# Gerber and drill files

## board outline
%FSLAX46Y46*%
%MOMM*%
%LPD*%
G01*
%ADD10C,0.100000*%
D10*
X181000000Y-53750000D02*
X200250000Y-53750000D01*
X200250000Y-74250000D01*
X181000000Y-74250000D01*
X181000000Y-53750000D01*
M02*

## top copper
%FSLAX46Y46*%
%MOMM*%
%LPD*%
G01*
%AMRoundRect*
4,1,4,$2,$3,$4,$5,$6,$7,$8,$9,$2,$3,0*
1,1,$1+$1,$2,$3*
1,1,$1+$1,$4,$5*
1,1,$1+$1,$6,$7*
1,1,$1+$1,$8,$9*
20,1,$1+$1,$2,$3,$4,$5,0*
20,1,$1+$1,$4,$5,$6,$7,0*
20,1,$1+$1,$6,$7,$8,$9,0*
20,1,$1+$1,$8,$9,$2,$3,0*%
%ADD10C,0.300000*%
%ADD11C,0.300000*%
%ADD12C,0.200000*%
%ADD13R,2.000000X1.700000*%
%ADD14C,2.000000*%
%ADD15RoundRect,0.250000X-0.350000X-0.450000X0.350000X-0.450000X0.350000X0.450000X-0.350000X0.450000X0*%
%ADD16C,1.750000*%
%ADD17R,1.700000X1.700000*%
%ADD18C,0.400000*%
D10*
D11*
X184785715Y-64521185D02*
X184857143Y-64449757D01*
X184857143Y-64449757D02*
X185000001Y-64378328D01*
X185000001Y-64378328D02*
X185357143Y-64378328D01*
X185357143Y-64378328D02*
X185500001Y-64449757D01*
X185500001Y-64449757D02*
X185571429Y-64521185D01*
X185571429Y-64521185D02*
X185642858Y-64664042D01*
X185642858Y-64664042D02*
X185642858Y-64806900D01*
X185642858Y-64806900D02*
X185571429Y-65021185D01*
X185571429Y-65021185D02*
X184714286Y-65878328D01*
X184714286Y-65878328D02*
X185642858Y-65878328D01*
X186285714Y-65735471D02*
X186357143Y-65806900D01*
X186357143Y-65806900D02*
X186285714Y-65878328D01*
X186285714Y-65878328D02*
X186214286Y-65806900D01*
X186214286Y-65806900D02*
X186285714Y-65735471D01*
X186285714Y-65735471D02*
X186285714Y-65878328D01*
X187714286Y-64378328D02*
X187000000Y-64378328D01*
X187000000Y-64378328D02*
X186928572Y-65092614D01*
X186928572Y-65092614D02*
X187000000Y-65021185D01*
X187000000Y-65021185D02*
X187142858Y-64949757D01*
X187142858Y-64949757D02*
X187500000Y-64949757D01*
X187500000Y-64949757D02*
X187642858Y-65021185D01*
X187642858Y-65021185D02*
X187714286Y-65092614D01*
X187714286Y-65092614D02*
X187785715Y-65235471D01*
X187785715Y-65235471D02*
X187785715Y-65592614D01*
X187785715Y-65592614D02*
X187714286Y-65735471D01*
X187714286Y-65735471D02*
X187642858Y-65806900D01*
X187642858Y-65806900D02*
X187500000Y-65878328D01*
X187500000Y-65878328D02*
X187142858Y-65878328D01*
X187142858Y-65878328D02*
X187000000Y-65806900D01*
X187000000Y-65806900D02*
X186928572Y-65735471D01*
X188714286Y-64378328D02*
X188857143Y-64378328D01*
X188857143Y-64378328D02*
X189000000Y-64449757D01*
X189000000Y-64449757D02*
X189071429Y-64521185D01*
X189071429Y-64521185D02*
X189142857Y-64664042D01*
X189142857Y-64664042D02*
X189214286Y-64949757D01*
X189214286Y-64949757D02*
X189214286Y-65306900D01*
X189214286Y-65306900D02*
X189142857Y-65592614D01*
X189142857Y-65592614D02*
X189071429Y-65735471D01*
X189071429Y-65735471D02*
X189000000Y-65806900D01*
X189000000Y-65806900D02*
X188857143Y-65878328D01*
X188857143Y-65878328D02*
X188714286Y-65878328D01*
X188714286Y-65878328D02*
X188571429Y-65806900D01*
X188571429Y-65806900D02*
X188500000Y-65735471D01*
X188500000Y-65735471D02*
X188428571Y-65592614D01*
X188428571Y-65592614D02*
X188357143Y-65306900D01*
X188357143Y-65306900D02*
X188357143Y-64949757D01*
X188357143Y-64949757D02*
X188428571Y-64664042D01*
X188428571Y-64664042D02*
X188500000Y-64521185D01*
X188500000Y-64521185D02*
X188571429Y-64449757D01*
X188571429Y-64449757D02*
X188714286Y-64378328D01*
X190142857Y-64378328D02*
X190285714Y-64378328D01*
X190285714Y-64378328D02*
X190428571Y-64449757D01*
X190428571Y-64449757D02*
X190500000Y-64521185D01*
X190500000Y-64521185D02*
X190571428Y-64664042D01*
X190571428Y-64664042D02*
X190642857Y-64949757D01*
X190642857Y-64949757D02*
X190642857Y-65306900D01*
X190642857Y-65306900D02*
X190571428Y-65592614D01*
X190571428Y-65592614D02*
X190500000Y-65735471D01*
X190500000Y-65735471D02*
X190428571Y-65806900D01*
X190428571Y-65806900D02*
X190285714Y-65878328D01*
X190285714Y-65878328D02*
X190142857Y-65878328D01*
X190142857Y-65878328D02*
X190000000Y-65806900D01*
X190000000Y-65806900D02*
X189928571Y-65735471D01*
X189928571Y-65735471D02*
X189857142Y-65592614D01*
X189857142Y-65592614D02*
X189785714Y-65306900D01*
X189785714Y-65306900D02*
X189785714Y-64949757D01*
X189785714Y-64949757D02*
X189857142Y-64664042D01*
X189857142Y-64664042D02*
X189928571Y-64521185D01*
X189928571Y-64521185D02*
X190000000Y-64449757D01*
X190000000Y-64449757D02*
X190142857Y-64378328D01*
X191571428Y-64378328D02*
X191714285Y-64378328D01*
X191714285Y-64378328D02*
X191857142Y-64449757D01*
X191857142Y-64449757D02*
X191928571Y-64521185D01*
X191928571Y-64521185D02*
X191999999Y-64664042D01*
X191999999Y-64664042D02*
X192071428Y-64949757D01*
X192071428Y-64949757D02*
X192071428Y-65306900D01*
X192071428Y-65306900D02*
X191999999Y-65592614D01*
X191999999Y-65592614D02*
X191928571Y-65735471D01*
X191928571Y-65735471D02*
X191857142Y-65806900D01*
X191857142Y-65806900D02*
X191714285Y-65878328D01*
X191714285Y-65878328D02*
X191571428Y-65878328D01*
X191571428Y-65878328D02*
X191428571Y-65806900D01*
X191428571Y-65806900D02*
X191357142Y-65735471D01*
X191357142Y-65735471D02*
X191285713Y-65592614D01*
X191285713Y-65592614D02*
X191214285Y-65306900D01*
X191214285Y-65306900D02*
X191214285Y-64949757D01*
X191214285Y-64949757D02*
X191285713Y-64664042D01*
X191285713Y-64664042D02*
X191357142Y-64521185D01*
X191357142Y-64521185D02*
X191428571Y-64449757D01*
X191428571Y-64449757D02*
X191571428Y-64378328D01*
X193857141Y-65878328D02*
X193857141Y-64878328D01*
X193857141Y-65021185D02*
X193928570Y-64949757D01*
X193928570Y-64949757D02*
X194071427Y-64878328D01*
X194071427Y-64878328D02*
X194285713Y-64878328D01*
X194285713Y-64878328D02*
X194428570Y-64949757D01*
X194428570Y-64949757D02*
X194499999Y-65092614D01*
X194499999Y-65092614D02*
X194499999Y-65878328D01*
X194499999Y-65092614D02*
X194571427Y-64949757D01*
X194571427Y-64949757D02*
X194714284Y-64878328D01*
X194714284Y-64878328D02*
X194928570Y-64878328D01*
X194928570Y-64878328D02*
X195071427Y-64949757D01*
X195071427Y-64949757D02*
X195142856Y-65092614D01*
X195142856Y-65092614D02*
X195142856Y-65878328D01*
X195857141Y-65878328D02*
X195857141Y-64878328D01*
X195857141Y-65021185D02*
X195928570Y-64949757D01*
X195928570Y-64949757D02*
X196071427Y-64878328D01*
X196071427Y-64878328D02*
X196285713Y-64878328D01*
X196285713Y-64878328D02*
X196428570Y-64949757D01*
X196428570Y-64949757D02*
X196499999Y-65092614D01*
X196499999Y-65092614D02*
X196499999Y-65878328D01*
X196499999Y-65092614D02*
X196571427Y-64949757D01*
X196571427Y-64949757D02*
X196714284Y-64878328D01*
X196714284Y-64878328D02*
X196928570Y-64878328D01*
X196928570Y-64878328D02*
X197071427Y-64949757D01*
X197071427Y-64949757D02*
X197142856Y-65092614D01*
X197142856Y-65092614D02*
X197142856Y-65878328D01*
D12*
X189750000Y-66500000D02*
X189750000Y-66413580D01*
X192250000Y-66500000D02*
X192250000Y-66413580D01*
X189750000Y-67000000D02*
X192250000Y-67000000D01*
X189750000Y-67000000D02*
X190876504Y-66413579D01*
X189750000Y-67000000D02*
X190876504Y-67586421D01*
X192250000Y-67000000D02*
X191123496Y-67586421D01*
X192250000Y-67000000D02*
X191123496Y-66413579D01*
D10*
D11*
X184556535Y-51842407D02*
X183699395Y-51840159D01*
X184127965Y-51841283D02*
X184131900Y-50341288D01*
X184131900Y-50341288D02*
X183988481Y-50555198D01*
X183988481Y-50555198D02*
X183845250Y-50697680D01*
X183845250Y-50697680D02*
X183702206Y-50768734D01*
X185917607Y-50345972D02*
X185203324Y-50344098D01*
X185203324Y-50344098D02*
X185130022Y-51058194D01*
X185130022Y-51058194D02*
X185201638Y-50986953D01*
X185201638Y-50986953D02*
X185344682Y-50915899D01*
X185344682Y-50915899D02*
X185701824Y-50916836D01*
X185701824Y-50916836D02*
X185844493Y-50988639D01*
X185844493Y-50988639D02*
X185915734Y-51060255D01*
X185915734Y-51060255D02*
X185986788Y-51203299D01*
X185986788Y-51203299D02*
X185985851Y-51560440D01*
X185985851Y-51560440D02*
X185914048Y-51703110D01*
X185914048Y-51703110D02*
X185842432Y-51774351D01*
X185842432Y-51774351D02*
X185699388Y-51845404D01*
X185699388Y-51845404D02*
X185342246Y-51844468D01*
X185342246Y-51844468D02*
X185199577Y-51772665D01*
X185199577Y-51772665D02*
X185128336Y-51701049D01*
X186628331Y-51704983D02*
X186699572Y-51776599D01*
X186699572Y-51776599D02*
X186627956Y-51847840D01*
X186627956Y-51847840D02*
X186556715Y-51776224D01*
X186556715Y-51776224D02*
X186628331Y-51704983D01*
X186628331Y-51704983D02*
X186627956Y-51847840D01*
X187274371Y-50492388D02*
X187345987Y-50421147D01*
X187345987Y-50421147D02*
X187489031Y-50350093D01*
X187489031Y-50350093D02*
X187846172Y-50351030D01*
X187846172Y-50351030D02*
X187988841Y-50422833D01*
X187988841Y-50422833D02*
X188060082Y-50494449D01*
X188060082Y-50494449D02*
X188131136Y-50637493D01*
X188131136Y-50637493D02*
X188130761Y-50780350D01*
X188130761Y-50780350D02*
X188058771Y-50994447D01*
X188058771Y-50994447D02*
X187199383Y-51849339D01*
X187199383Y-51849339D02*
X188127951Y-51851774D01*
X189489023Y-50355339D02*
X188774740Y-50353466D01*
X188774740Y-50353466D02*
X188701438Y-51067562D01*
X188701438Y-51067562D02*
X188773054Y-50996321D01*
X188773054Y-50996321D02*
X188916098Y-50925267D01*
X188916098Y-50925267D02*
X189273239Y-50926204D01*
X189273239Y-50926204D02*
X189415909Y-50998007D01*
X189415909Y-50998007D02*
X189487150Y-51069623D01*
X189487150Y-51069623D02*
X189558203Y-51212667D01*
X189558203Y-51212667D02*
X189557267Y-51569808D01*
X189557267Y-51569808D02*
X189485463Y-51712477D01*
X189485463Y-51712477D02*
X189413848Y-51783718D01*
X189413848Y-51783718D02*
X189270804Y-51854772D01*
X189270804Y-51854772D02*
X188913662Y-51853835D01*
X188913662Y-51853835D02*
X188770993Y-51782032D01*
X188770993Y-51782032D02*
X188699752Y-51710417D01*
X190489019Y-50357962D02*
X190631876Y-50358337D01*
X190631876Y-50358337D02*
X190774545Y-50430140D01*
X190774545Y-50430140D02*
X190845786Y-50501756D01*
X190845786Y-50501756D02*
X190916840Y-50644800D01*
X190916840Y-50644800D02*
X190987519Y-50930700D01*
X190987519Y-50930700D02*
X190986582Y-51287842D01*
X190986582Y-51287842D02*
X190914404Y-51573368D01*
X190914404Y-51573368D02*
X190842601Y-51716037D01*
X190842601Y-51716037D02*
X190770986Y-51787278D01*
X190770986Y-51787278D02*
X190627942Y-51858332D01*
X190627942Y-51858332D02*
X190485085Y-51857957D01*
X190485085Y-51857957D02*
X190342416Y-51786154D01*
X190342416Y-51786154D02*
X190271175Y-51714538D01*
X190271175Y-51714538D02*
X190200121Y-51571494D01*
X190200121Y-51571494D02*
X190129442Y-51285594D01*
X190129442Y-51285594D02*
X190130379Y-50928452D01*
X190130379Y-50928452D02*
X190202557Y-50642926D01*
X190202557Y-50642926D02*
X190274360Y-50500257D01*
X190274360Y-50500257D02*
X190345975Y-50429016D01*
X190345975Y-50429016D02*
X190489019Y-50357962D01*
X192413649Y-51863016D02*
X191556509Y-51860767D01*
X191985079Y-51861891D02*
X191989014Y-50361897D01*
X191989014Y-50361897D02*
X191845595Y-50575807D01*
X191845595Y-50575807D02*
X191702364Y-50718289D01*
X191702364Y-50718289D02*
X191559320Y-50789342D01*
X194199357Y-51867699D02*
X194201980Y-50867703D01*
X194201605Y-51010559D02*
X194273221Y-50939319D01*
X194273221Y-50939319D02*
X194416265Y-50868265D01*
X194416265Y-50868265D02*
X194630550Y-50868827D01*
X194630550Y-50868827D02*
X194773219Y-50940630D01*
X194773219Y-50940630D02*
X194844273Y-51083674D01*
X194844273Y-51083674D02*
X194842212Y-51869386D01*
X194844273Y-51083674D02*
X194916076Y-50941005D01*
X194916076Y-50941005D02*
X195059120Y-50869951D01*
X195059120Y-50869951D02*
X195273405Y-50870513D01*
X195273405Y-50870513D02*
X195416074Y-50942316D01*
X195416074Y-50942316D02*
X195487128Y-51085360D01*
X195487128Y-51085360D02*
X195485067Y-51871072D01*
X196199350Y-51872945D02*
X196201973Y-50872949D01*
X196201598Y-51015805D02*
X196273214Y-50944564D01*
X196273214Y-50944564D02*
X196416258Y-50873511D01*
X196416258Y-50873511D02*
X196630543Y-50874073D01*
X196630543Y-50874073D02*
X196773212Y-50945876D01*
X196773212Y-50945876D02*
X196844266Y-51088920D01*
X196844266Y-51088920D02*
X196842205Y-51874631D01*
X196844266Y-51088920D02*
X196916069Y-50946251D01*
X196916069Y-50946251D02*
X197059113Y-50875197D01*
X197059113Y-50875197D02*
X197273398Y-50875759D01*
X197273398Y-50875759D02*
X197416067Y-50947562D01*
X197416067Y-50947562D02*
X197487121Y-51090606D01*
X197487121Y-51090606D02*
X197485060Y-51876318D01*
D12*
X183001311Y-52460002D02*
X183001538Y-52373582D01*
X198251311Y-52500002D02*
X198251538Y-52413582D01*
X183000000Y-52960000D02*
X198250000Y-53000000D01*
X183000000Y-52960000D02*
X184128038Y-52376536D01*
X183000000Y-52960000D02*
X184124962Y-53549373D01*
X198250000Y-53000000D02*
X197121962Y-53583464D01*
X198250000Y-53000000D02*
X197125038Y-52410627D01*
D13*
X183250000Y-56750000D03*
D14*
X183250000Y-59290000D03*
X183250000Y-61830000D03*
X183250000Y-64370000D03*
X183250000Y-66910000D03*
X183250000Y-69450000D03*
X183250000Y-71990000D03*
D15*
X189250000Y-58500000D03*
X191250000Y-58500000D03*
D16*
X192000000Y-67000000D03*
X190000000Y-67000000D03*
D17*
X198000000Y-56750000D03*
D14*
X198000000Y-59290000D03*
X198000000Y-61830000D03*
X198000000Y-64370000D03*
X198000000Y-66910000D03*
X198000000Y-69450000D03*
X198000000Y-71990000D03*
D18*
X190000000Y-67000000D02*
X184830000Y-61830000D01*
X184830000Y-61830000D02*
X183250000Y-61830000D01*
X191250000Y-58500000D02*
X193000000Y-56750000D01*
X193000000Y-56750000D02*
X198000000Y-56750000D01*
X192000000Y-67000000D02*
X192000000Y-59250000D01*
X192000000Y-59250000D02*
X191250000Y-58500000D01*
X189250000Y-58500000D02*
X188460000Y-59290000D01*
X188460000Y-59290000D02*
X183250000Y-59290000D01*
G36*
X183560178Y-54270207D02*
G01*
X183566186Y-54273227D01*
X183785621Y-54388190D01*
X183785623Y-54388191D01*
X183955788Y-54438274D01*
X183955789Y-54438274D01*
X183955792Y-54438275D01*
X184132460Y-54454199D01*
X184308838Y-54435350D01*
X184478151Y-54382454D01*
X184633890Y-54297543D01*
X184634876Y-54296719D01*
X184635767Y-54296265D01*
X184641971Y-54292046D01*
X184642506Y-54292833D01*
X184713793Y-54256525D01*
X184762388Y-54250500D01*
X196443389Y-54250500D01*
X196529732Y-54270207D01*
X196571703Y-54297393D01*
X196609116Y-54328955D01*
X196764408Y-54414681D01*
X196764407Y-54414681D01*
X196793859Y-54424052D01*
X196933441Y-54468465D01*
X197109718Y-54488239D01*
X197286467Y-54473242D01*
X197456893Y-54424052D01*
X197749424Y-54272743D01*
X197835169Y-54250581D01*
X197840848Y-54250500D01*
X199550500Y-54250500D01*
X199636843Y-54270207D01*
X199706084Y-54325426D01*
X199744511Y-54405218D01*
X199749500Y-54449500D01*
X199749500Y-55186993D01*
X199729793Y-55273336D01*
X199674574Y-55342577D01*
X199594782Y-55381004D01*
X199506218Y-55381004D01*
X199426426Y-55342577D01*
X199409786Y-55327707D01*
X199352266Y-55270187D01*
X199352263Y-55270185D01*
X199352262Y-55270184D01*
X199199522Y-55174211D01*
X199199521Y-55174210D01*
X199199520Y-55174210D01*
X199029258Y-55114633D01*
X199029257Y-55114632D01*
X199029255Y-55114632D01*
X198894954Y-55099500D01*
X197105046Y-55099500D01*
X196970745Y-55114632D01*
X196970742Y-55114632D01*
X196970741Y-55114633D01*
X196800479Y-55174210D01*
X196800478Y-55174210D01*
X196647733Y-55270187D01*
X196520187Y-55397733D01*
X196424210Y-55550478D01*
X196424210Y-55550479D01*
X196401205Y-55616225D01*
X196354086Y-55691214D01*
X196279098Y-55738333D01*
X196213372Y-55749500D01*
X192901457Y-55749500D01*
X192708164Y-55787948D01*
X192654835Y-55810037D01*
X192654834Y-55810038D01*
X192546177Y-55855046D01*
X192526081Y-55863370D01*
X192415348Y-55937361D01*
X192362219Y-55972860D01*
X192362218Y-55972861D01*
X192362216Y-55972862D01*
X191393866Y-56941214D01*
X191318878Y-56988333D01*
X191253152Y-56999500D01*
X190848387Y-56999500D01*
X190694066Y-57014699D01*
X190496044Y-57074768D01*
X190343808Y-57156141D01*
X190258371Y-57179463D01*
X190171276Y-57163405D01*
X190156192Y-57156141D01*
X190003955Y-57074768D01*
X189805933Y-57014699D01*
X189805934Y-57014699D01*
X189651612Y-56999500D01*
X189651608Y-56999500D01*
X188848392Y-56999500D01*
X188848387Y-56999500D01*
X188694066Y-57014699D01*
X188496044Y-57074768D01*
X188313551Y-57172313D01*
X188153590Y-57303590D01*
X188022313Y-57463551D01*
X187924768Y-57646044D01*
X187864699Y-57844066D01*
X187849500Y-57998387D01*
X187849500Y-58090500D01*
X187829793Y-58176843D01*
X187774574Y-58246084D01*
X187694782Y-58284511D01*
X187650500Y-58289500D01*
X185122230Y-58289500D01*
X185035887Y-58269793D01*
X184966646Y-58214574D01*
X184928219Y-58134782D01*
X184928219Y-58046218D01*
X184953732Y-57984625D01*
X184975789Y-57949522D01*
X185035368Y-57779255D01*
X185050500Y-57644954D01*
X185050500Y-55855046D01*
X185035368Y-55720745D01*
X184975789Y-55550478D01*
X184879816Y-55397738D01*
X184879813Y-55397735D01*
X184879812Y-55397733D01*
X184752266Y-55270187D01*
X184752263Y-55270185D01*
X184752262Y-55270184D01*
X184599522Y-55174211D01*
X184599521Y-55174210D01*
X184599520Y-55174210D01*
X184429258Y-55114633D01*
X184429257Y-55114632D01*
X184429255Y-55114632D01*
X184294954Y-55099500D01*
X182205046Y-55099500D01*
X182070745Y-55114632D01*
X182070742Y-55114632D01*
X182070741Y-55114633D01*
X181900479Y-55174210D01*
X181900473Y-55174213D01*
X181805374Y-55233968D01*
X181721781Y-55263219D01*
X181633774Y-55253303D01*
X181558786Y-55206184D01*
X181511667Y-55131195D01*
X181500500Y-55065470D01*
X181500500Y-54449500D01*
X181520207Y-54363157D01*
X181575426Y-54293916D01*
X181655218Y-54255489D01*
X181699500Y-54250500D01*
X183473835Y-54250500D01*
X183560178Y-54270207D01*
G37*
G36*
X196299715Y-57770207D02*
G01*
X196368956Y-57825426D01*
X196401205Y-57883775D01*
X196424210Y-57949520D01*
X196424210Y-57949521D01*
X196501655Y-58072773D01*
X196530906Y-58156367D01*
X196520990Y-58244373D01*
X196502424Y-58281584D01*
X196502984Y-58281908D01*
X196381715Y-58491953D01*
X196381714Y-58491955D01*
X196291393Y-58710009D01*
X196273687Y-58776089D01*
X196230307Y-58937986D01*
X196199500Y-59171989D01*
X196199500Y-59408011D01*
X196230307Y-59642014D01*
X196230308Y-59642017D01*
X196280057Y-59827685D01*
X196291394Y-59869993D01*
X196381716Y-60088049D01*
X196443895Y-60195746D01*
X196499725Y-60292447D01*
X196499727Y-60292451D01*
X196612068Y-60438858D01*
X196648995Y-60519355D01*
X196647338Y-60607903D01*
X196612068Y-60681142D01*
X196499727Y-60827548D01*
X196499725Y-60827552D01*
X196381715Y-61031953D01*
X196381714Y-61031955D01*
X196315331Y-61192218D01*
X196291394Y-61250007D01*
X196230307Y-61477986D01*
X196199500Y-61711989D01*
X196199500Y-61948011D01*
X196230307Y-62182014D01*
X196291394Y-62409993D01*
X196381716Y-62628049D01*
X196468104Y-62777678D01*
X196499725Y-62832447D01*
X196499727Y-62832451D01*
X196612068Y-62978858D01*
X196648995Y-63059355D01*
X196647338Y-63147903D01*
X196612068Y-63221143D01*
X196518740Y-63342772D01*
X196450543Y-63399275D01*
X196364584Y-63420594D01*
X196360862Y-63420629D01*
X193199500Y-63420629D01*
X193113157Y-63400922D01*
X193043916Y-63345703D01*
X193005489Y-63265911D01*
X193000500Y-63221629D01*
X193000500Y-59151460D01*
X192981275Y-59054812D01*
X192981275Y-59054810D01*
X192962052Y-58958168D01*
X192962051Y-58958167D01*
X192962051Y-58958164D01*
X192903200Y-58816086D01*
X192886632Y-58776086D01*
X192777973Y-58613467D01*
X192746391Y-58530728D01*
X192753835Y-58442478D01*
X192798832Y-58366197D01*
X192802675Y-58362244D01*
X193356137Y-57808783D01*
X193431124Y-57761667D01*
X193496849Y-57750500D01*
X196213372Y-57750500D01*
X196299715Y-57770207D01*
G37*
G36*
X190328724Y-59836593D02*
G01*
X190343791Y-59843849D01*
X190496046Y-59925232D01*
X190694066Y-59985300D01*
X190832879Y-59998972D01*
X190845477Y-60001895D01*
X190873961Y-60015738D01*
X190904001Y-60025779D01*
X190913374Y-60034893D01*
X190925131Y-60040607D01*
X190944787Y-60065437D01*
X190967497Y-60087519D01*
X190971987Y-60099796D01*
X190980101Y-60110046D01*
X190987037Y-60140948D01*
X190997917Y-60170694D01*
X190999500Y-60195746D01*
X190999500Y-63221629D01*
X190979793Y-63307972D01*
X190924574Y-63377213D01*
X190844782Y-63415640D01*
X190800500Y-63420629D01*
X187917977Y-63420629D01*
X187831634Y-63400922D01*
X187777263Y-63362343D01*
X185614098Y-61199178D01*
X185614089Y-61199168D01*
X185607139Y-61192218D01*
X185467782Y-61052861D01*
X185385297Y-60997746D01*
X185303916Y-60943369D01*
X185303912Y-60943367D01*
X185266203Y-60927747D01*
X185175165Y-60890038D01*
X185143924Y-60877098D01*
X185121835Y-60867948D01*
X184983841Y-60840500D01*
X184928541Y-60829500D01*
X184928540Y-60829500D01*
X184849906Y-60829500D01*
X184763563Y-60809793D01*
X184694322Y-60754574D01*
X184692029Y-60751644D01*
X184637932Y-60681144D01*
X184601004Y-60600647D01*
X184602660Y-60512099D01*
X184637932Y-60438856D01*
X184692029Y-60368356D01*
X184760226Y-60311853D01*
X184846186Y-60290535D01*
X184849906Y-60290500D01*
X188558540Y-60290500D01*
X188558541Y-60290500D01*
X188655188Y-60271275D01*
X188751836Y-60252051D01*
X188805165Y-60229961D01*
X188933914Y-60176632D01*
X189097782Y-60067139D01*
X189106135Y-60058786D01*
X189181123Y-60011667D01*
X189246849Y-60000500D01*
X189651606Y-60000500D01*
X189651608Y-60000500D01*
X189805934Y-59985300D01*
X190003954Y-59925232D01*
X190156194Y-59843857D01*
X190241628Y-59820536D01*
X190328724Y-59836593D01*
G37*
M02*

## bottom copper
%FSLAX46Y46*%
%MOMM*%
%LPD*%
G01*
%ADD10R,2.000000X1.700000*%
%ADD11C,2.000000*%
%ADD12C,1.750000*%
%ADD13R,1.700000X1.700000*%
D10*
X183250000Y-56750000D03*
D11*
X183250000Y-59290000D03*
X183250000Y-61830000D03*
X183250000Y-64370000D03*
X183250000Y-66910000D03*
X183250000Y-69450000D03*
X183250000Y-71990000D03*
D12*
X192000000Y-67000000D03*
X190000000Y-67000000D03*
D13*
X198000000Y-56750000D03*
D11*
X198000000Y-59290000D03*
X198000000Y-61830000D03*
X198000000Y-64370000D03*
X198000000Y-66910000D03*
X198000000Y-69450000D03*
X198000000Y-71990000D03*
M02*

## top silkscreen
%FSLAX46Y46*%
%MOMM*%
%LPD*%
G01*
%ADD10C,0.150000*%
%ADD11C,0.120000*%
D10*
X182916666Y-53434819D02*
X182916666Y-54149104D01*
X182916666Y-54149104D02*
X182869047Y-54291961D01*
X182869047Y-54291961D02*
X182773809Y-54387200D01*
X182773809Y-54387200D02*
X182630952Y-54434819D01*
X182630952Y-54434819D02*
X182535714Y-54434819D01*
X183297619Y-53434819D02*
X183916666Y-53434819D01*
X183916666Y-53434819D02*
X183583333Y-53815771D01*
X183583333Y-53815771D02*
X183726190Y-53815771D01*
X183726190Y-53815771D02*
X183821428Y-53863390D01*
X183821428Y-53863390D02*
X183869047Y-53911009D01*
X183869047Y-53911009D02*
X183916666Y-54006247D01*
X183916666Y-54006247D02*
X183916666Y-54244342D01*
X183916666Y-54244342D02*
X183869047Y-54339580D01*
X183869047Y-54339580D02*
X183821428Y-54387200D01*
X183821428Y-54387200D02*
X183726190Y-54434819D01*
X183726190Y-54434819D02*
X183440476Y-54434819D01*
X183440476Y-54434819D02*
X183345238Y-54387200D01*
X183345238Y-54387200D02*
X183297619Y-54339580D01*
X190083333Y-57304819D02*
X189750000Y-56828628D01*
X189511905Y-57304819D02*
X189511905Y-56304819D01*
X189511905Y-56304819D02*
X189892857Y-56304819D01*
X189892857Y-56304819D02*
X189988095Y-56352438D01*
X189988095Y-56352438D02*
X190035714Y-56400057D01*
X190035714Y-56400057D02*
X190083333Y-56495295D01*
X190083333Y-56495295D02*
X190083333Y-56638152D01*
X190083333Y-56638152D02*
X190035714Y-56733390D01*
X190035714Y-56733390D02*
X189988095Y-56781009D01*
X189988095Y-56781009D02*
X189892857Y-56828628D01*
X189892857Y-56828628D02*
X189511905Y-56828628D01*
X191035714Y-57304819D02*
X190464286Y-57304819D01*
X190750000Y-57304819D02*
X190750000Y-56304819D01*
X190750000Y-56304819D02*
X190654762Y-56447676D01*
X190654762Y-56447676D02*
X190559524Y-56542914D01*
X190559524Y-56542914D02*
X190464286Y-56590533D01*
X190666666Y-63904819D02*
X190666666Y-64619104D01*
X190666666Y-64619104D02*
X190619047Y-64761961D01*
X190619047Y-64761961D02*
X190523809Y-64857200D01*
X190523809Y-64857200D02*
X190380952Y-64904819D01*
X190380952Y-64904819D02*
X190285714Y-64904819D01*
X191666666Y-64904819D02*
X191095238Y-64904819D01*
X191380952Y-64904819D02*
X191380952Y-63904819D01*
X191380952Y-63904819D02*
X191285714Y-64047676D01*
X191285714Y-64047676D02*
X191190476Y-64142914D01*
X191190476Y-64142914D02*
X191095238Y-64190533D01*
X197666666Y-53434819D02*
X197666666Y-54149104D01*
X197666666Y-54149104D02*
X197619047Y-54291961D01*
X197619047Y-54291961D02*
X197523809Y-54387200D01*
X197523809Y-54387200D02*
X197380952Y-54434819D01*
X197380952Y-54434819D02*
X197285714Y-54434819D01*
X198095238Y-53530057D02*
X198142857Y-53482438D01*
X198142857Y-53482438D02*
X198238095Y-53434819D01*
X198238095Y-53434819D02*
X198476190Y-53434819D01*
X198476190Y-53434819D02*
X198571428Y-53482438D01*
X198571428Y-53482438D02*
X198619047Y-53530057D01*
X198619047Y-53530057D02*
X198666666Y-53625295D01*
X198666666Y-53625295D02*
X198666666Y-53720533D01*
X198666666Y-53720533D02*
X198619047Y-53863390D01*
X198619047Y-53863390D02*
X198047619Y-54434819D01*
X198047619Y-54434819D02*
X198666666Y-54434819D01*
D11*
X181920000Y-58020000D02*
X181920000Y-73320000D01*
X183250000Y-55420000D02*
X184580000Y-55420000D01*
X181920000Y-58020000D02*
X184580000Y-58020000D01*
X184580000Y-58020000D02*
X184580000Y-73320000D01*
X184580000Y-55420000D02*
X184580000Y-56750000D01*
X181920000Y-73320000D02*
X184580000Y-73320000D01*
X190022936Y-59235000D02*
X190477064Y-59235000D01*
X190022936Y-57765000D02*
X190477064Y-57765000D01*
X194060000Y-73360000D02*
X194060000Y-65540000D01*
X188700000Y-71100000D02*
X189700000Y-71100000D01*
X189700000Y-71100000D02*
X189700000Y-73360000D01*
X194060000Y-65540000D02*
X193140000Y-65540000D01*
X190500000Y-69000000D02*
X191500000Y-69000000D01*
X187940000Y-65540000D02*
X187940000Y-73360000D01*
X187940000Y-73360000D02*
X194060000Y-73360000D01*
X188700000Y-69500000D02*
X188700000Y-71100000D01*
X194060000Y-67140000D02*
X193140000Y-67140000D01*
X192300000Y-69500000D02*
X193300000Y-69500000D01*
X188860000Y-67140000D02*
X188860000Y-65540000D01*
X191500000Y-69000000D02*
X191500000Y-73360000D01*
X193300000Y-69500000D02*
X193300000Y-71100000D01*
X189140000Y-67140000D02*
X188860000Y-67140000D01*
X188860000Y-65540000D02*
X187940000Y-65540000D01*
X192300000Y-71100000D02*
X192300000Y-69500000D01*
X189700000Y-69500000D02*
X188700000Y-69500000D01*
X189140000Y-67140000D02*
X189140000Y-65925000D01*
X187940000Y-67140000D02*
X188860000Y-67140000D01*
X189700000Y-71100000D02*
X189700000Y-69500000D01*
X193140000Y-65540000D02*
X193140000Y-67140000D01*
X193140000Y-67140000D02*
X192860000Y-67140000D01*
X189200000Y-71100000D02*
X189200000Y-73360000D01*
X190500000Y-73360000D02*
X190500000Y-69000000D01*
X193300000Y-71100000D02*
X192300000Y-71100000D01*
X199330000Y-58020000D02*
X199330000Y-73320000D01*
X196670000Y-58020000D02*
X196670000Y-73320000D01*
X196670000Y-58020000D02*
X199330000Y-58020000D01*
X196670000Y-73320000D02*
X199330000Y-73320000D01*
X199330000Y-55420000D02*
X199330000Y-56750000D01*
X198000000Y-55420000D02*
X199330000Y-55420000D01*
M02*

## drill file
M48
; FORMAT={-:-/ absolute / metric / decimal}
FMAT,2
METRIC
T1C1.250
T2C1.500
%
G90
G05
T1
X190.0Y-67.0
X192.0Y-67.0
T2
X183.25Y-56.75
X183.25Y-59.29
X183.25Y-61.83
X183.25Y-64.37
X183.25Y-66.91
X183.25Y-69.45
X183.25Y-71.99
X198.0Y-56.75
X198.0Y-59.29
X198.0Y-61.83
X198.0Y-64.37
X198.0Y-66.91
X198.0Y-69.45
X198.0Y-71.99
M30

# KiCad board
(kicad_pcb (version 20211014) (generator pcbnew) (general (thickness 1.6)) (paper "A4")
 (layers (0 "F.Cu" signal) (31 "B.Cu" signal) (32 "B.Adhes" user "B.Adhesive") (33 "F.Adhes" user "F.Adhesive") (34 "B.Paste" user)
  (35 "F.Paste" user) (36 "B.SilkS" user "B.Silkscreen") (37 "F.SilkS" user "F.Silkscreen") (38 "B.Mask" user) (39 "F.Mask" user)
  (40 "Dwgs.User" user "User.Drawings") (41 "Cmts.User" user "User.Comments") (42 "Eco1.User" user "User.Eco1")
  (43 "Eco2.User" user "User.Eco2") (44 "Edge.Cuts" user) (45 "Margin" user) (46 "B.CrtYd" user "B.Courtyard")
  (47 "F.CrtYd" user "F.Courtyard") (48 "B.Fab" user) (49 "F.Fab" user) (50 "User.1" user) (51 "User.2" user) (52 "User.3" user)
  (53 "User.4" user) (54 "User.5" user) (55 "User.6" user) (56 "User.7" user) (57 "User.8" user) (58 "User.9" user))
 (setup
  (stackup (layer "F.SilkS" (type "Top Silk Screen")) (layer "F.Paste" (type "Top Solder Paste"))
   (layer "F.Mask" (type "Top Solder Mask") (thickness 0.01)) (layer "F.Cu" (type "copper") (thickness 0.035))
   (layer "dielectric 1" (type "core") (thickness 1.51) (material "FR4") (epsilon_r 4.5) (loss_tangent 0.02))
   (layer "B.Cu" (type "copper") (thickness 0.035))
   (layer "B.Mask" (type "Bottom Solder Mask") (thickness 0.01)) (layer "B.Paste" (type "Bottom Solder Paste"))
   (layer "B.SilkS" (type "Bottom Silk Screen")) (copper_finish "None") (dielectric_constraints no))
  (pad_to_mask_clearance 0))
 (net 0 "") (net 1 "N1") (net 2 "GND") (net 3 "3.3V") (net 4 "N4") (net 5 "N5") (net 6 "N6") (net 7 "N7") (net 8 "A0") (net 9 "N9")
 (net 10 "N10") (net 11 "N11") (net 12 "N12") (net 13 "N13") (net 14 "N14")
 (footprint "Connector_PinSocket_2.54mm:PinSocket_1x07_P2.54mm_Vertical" (layer "F.Cu") (at 183.25 56.75)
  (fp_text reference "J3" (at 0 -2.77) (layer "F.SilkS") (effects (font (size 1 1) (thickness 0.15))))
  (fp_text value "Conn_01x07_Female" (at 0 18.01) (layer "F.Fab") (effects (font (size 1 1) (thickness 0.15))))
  (fp_line (start -1.33 1.27) (end -1.33 16.57) (layer "F.SilkS") (width 0.12))
  (fp_line (start 0 -1.33) (end 1.33 -1.33) (layer "F.SilkS") (width 0.12))
  (fp_line (start -1.33 1.27) (end 1.33 1.27) (layer "F.SilkS") (width 0.12))
  (fp_line (start 1.33 1.27) (end 1.33 16.57) (layer "F.SilkS") (width 0.12))
  (fp_line (start 1.33 -1.33) (end 1.33 0) (layer "F.SilkS") (width 0.12))
  (fp_line (start -1.33 16.57) (end 1.33 16.57) (layer "F.SilkS") (width 0.12))
  (pad "1" thru_hole rect (at 0 0) (size 2 1.7) (drill 1.5) (layers *.Cu *.Mask) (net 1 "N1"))
  (pad "2" thru_hole circle (at 0 2.54) (size 2 2) (drill 1.5) (layers *.Cu *.Mask) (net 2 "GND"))
  (pad "3" thru_hole circle (at 0 5.08) (size 2 2) (drill 1.5) (layers *.Cu *.Mask) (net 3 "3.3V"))
  (pad "4" thru_hole circle (at 0 7.62) (size 2 2) (drill 1.5) (layers *.Cu *.Mask) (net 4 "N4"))
  (pad "5" thru_hole circle (at 0 10.16) (size 2 2) (drill 1.5) (layers *.Cu *.Mask) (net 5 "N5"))
  (pad "6" thru_hole circle (at 0 12.7) (size 2 2) (drill 1.5) (layers *.Cu *.Mask) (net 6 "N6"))
  (pad "7" thru_hole circle (at 0 15.24) (size 2 2) (drill 1.5) (layers *.Cu *.Mask) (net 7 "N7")))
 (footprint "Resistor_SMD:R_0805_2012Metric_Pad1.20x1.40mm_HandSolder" (layer "F.Cu") (at 190.25 58.5)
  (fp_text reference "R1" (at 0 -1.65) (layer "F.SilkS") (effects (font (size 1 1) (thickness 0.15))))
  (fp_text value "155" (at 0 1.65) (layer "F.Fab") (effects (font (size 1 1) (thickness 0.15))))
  (fp_line (start -0.227064 0.735) (end 0.227064 0.735) (layer "F.SilkS") (width 0.12))
  (fp_line (start -0.227064 -0.735) (end 0.227064 -0.735) (layer "F.SilkS") (width 0.12))
  (pad "1" smd roundrect (at -1 0) (size 1.2 1.4) (layers "F.Cu" "F.Paste" "F.Mask") (roundrect_rratio 0.2083333333) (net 2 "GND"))
  (pad "2" smd roundrect (at 1 0) (size 1.2 1.4) (layers "F.Cu" "F.Paste" "F.Mask") (roundrect_rratio 0.2083333333) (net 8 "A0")))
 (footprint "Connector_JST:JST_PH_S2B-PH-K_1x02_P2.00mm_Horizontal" (layer "F.Cu") (at 190 67)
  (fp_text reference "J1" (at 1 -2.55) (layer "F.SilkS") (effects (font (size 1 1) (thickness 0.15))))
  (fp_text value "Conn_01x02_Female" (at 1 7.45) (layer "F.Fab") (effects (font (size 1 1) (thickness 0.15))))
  (fp_line (start 4.06 6.36) (end 4.06 -1.46) (layer "F.SilkS") (width 0.12))
  (fp_line (start -1.3 4.1) (end -0.3 4.1) (layer "F.SilkS") (width 0.12))
  (fp_line (start -0.3 4.1) (end -0.3 6.36) (layer "F.SilkS") (width 0.12))
  (fp_line (start 4.06 -1.46) (end 3.14 -1.46) (layer "F.SilkS") (width 0.12))
  (fp_line (start 0.5 2) (end 1.5 2) (layer "F.SilkS") (width 0.12))
  (fp_line (start -2.06 -1.46) (end -2.06 6.36) (layer "F.SilkS") (width 0.12))
  (fp_line (start -2.06 6.36) (end 4.06 6.36) (layer "F.SilkS") (width 0.12))
  (fp_line (start -1.3 2.5) (end -1.3 4.1) (layer "F.SilkS") (width 0.12))
  (fp_line (start 4.06 0.14) (end 3.14 0.14) (layer "F.SilkS") (width 0.12))
  (fp_line (start 2.3 2.5) (end 3.3 2.5) (layer "F.SilkS") (width 0.12))
  (fp_line (start -1.14 0.14) (end -1.14 -1.46) (layer "F.SilkS") (width 0.12))
  (fp_line (start 1.5 2) (end 1.5 6.36) (layer "F.SilkS") (width 0.12))
  (fp_line (start 3.3 2.5) (end 3.3 4.1) (layer "F.SilkS") (width 0.12))
  (fp_line (start -0.86 0.14) (end -1.14 0.14) (layer "F.SilkS") (width 0.12))
  (fp_line (start -1.14 -1.46) (end -2.06 -1.46) (layer "F.SilkS") (width 0.12))
  (fp_line (start 2.3 4.1) (end 2.3 2.5) (layer "F.SilkS") (width 0.12))
  (fp_line (start -0.3 2.5) (end -1.3 2.5) (layer "F.SilkS") (width 0.12))
  (fp_line (start -0.86 0.14) (end -0.86 -1.075) (layer "F.SilkS") (width 0.12))
  (fp_line (start -2.06 0.14) (end -1.14 0.14) (layer "F.SilkS") (width 0.12))
  (fp_line (start -0.3 4.1) (end -0.3 2.5) (layer "F.SilkS") (width 0.12))
  (fp_line (start 3.14 -1.46) (end 3.14 0.14) (layer "F.SilkS") (width 0.12))
  (fp_line (start 3.14 0.14) (end 2.86 0.14) (layer "F.SilkS") (width 0.12))
  (fp_line (start -0.8 4.1) (end -0.8 6.36) (layer "F.SilkS") (width 0.12))
  (fp_line (start 0.5 6.36) (end 0.5 2) (layer "F.SilkS") (width 0.12))
  (fp_line (start 3.3 4.1) (end 2.3 4.1) (layer "F.SilkS") (width 0.12))
  (pad "" thru_hole circle (at 2 0) (size 1.75 1.75) (drill 1.25) (layers *.Cu *.Mask) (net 8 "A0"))
  (pad "1" thru_hole circle (at 0 0) (size 1.75 1.75) (drill 1.25) (layers *.Cu *.Mask) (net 3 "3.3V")))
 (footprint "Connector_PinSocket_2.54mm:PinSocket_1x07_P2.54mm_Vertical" (layer "F.Cu") (at 198 56.75)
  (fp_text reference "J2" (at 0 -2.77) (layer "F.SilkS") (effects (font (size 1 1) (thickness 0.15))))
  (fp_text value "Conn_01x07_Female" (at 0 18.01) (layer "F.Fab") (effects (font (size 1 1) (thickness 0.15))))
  (fp_line (start 1.33 1.27) (end 1.33 16.57) (layer "F.SilkS") (width 0.12))
  (fp_line (start -1.33 1.27) (end -1.33 16.57) (layer "F.SilkS") (width 0.12))
  (fp_line (start -1.33 1.27) (end 1.33 1.27) (layer "F.SilkS") (width 0.12))
  (fp_line (start -1.33 16.57) (end 1.33 16.57) (layer "F.SilkS") (width 0.12))
  (fp_line (start 1.33 -1.33) (end 1.33 0) (layer "F.SilkS") (width 0.12))
  (fp_line (start 0 -1.33) (end 1.33 -1.33) (layer "F.SilkS") (width 0.12))
  (pad "1" thru_hole rect (at 0 0) (size 1.7 1.7) (drill 1.5) (layers *.Cu *.Mask) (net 8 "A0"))
  (pad "2" thru_hole circle (at 0 2.54) (size 2 2) (drill 1.5) (layers *.Cu *.Mask) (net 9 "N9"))
  (pad "3" thru_hole circle (at 0 5.08) (size 2 2) (drill 1.5) (layers *.Cu *.Mask) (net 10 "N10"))
  (pad "4" thru_hole circle (at 0 7.62) (size 2 2) (drill 1.5) (layers *.Cu *.Mask) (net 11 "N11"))
  (pad "5" thru_hole circle (at 0 10.16) (size 2 2) (drill 1.5) (layers *.Cu *.Mask) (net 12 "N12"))
  (pad "6" thru_hole circle (at 0 12.7) (size 2 2) (drill 1.5) (layers *.Cu *.Mask) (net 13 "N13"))
  (pad "7" thru_hole circle (at 0 15.24) (size 2 2) (drill 1.5) (layers *.Cu *.Mask) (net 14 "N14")))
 (gr_rect (start 181 53.75) (end 200.25 74.25) (layer "Edge.Cuts") (width 0.1) (fill none))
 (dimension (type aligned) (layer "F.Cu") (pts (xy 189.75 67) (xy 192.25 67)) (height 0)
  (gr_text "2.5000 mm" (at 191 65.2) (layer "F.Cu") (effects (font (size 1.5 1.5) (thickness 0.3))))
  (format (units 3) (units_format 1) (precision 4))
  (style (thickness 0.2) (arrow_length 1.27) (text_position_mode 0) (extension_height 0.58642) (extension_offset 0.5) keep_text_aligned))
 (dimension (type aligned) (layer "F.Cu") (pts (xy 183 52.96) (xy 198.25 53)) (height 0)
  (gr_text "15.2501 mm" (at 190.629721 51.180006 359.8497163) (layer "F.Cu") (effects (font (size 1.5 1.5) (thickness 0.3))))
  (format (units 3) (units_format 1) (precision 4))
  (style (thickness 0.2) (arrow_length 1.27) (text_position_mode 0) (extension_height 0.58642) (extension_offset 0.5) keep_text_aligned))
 (segment (start 190 67) (end 184.83 61.83) (width 0.4) (layer "F.Cu") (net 3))
 (segment (start 184.83 61.83) (end 183.25 61.83) (width 0.4) (layer "F.Cu") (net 3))
 (segment (start 191.25 58.5) (end 193 56.75) (width 0.4) (layer "F.Cu") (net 8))
 (segment (start 193 56.75) (end 198 56.75) (width 0.4) (layer "F.Cu") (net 8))
 (segment (start 192 67) (end 192 59.25) (width 0.4) (layer "F.Cu") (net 8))
 (segment (start 192 59.25) (end 191.25 58.5) (width 0.4) (layer "F.Cu") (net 8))
 (segment (start 189.25 58.5) (end 188.46 59.29) (width 0.4) (layer "F.Cu") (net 2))
 (segment (start 188.46 59.29) (end 183.25 59.29) (width 0.4) (layer "F.Cu") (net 2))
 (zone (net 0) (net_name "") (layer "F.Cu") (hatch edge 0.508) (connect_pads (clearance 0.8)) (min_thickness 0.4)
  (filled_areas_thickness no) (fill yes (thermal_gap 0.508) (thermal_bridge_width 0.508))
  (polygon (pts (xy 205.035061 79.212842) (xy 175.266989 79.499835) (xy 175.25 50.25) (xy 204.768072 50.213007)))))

